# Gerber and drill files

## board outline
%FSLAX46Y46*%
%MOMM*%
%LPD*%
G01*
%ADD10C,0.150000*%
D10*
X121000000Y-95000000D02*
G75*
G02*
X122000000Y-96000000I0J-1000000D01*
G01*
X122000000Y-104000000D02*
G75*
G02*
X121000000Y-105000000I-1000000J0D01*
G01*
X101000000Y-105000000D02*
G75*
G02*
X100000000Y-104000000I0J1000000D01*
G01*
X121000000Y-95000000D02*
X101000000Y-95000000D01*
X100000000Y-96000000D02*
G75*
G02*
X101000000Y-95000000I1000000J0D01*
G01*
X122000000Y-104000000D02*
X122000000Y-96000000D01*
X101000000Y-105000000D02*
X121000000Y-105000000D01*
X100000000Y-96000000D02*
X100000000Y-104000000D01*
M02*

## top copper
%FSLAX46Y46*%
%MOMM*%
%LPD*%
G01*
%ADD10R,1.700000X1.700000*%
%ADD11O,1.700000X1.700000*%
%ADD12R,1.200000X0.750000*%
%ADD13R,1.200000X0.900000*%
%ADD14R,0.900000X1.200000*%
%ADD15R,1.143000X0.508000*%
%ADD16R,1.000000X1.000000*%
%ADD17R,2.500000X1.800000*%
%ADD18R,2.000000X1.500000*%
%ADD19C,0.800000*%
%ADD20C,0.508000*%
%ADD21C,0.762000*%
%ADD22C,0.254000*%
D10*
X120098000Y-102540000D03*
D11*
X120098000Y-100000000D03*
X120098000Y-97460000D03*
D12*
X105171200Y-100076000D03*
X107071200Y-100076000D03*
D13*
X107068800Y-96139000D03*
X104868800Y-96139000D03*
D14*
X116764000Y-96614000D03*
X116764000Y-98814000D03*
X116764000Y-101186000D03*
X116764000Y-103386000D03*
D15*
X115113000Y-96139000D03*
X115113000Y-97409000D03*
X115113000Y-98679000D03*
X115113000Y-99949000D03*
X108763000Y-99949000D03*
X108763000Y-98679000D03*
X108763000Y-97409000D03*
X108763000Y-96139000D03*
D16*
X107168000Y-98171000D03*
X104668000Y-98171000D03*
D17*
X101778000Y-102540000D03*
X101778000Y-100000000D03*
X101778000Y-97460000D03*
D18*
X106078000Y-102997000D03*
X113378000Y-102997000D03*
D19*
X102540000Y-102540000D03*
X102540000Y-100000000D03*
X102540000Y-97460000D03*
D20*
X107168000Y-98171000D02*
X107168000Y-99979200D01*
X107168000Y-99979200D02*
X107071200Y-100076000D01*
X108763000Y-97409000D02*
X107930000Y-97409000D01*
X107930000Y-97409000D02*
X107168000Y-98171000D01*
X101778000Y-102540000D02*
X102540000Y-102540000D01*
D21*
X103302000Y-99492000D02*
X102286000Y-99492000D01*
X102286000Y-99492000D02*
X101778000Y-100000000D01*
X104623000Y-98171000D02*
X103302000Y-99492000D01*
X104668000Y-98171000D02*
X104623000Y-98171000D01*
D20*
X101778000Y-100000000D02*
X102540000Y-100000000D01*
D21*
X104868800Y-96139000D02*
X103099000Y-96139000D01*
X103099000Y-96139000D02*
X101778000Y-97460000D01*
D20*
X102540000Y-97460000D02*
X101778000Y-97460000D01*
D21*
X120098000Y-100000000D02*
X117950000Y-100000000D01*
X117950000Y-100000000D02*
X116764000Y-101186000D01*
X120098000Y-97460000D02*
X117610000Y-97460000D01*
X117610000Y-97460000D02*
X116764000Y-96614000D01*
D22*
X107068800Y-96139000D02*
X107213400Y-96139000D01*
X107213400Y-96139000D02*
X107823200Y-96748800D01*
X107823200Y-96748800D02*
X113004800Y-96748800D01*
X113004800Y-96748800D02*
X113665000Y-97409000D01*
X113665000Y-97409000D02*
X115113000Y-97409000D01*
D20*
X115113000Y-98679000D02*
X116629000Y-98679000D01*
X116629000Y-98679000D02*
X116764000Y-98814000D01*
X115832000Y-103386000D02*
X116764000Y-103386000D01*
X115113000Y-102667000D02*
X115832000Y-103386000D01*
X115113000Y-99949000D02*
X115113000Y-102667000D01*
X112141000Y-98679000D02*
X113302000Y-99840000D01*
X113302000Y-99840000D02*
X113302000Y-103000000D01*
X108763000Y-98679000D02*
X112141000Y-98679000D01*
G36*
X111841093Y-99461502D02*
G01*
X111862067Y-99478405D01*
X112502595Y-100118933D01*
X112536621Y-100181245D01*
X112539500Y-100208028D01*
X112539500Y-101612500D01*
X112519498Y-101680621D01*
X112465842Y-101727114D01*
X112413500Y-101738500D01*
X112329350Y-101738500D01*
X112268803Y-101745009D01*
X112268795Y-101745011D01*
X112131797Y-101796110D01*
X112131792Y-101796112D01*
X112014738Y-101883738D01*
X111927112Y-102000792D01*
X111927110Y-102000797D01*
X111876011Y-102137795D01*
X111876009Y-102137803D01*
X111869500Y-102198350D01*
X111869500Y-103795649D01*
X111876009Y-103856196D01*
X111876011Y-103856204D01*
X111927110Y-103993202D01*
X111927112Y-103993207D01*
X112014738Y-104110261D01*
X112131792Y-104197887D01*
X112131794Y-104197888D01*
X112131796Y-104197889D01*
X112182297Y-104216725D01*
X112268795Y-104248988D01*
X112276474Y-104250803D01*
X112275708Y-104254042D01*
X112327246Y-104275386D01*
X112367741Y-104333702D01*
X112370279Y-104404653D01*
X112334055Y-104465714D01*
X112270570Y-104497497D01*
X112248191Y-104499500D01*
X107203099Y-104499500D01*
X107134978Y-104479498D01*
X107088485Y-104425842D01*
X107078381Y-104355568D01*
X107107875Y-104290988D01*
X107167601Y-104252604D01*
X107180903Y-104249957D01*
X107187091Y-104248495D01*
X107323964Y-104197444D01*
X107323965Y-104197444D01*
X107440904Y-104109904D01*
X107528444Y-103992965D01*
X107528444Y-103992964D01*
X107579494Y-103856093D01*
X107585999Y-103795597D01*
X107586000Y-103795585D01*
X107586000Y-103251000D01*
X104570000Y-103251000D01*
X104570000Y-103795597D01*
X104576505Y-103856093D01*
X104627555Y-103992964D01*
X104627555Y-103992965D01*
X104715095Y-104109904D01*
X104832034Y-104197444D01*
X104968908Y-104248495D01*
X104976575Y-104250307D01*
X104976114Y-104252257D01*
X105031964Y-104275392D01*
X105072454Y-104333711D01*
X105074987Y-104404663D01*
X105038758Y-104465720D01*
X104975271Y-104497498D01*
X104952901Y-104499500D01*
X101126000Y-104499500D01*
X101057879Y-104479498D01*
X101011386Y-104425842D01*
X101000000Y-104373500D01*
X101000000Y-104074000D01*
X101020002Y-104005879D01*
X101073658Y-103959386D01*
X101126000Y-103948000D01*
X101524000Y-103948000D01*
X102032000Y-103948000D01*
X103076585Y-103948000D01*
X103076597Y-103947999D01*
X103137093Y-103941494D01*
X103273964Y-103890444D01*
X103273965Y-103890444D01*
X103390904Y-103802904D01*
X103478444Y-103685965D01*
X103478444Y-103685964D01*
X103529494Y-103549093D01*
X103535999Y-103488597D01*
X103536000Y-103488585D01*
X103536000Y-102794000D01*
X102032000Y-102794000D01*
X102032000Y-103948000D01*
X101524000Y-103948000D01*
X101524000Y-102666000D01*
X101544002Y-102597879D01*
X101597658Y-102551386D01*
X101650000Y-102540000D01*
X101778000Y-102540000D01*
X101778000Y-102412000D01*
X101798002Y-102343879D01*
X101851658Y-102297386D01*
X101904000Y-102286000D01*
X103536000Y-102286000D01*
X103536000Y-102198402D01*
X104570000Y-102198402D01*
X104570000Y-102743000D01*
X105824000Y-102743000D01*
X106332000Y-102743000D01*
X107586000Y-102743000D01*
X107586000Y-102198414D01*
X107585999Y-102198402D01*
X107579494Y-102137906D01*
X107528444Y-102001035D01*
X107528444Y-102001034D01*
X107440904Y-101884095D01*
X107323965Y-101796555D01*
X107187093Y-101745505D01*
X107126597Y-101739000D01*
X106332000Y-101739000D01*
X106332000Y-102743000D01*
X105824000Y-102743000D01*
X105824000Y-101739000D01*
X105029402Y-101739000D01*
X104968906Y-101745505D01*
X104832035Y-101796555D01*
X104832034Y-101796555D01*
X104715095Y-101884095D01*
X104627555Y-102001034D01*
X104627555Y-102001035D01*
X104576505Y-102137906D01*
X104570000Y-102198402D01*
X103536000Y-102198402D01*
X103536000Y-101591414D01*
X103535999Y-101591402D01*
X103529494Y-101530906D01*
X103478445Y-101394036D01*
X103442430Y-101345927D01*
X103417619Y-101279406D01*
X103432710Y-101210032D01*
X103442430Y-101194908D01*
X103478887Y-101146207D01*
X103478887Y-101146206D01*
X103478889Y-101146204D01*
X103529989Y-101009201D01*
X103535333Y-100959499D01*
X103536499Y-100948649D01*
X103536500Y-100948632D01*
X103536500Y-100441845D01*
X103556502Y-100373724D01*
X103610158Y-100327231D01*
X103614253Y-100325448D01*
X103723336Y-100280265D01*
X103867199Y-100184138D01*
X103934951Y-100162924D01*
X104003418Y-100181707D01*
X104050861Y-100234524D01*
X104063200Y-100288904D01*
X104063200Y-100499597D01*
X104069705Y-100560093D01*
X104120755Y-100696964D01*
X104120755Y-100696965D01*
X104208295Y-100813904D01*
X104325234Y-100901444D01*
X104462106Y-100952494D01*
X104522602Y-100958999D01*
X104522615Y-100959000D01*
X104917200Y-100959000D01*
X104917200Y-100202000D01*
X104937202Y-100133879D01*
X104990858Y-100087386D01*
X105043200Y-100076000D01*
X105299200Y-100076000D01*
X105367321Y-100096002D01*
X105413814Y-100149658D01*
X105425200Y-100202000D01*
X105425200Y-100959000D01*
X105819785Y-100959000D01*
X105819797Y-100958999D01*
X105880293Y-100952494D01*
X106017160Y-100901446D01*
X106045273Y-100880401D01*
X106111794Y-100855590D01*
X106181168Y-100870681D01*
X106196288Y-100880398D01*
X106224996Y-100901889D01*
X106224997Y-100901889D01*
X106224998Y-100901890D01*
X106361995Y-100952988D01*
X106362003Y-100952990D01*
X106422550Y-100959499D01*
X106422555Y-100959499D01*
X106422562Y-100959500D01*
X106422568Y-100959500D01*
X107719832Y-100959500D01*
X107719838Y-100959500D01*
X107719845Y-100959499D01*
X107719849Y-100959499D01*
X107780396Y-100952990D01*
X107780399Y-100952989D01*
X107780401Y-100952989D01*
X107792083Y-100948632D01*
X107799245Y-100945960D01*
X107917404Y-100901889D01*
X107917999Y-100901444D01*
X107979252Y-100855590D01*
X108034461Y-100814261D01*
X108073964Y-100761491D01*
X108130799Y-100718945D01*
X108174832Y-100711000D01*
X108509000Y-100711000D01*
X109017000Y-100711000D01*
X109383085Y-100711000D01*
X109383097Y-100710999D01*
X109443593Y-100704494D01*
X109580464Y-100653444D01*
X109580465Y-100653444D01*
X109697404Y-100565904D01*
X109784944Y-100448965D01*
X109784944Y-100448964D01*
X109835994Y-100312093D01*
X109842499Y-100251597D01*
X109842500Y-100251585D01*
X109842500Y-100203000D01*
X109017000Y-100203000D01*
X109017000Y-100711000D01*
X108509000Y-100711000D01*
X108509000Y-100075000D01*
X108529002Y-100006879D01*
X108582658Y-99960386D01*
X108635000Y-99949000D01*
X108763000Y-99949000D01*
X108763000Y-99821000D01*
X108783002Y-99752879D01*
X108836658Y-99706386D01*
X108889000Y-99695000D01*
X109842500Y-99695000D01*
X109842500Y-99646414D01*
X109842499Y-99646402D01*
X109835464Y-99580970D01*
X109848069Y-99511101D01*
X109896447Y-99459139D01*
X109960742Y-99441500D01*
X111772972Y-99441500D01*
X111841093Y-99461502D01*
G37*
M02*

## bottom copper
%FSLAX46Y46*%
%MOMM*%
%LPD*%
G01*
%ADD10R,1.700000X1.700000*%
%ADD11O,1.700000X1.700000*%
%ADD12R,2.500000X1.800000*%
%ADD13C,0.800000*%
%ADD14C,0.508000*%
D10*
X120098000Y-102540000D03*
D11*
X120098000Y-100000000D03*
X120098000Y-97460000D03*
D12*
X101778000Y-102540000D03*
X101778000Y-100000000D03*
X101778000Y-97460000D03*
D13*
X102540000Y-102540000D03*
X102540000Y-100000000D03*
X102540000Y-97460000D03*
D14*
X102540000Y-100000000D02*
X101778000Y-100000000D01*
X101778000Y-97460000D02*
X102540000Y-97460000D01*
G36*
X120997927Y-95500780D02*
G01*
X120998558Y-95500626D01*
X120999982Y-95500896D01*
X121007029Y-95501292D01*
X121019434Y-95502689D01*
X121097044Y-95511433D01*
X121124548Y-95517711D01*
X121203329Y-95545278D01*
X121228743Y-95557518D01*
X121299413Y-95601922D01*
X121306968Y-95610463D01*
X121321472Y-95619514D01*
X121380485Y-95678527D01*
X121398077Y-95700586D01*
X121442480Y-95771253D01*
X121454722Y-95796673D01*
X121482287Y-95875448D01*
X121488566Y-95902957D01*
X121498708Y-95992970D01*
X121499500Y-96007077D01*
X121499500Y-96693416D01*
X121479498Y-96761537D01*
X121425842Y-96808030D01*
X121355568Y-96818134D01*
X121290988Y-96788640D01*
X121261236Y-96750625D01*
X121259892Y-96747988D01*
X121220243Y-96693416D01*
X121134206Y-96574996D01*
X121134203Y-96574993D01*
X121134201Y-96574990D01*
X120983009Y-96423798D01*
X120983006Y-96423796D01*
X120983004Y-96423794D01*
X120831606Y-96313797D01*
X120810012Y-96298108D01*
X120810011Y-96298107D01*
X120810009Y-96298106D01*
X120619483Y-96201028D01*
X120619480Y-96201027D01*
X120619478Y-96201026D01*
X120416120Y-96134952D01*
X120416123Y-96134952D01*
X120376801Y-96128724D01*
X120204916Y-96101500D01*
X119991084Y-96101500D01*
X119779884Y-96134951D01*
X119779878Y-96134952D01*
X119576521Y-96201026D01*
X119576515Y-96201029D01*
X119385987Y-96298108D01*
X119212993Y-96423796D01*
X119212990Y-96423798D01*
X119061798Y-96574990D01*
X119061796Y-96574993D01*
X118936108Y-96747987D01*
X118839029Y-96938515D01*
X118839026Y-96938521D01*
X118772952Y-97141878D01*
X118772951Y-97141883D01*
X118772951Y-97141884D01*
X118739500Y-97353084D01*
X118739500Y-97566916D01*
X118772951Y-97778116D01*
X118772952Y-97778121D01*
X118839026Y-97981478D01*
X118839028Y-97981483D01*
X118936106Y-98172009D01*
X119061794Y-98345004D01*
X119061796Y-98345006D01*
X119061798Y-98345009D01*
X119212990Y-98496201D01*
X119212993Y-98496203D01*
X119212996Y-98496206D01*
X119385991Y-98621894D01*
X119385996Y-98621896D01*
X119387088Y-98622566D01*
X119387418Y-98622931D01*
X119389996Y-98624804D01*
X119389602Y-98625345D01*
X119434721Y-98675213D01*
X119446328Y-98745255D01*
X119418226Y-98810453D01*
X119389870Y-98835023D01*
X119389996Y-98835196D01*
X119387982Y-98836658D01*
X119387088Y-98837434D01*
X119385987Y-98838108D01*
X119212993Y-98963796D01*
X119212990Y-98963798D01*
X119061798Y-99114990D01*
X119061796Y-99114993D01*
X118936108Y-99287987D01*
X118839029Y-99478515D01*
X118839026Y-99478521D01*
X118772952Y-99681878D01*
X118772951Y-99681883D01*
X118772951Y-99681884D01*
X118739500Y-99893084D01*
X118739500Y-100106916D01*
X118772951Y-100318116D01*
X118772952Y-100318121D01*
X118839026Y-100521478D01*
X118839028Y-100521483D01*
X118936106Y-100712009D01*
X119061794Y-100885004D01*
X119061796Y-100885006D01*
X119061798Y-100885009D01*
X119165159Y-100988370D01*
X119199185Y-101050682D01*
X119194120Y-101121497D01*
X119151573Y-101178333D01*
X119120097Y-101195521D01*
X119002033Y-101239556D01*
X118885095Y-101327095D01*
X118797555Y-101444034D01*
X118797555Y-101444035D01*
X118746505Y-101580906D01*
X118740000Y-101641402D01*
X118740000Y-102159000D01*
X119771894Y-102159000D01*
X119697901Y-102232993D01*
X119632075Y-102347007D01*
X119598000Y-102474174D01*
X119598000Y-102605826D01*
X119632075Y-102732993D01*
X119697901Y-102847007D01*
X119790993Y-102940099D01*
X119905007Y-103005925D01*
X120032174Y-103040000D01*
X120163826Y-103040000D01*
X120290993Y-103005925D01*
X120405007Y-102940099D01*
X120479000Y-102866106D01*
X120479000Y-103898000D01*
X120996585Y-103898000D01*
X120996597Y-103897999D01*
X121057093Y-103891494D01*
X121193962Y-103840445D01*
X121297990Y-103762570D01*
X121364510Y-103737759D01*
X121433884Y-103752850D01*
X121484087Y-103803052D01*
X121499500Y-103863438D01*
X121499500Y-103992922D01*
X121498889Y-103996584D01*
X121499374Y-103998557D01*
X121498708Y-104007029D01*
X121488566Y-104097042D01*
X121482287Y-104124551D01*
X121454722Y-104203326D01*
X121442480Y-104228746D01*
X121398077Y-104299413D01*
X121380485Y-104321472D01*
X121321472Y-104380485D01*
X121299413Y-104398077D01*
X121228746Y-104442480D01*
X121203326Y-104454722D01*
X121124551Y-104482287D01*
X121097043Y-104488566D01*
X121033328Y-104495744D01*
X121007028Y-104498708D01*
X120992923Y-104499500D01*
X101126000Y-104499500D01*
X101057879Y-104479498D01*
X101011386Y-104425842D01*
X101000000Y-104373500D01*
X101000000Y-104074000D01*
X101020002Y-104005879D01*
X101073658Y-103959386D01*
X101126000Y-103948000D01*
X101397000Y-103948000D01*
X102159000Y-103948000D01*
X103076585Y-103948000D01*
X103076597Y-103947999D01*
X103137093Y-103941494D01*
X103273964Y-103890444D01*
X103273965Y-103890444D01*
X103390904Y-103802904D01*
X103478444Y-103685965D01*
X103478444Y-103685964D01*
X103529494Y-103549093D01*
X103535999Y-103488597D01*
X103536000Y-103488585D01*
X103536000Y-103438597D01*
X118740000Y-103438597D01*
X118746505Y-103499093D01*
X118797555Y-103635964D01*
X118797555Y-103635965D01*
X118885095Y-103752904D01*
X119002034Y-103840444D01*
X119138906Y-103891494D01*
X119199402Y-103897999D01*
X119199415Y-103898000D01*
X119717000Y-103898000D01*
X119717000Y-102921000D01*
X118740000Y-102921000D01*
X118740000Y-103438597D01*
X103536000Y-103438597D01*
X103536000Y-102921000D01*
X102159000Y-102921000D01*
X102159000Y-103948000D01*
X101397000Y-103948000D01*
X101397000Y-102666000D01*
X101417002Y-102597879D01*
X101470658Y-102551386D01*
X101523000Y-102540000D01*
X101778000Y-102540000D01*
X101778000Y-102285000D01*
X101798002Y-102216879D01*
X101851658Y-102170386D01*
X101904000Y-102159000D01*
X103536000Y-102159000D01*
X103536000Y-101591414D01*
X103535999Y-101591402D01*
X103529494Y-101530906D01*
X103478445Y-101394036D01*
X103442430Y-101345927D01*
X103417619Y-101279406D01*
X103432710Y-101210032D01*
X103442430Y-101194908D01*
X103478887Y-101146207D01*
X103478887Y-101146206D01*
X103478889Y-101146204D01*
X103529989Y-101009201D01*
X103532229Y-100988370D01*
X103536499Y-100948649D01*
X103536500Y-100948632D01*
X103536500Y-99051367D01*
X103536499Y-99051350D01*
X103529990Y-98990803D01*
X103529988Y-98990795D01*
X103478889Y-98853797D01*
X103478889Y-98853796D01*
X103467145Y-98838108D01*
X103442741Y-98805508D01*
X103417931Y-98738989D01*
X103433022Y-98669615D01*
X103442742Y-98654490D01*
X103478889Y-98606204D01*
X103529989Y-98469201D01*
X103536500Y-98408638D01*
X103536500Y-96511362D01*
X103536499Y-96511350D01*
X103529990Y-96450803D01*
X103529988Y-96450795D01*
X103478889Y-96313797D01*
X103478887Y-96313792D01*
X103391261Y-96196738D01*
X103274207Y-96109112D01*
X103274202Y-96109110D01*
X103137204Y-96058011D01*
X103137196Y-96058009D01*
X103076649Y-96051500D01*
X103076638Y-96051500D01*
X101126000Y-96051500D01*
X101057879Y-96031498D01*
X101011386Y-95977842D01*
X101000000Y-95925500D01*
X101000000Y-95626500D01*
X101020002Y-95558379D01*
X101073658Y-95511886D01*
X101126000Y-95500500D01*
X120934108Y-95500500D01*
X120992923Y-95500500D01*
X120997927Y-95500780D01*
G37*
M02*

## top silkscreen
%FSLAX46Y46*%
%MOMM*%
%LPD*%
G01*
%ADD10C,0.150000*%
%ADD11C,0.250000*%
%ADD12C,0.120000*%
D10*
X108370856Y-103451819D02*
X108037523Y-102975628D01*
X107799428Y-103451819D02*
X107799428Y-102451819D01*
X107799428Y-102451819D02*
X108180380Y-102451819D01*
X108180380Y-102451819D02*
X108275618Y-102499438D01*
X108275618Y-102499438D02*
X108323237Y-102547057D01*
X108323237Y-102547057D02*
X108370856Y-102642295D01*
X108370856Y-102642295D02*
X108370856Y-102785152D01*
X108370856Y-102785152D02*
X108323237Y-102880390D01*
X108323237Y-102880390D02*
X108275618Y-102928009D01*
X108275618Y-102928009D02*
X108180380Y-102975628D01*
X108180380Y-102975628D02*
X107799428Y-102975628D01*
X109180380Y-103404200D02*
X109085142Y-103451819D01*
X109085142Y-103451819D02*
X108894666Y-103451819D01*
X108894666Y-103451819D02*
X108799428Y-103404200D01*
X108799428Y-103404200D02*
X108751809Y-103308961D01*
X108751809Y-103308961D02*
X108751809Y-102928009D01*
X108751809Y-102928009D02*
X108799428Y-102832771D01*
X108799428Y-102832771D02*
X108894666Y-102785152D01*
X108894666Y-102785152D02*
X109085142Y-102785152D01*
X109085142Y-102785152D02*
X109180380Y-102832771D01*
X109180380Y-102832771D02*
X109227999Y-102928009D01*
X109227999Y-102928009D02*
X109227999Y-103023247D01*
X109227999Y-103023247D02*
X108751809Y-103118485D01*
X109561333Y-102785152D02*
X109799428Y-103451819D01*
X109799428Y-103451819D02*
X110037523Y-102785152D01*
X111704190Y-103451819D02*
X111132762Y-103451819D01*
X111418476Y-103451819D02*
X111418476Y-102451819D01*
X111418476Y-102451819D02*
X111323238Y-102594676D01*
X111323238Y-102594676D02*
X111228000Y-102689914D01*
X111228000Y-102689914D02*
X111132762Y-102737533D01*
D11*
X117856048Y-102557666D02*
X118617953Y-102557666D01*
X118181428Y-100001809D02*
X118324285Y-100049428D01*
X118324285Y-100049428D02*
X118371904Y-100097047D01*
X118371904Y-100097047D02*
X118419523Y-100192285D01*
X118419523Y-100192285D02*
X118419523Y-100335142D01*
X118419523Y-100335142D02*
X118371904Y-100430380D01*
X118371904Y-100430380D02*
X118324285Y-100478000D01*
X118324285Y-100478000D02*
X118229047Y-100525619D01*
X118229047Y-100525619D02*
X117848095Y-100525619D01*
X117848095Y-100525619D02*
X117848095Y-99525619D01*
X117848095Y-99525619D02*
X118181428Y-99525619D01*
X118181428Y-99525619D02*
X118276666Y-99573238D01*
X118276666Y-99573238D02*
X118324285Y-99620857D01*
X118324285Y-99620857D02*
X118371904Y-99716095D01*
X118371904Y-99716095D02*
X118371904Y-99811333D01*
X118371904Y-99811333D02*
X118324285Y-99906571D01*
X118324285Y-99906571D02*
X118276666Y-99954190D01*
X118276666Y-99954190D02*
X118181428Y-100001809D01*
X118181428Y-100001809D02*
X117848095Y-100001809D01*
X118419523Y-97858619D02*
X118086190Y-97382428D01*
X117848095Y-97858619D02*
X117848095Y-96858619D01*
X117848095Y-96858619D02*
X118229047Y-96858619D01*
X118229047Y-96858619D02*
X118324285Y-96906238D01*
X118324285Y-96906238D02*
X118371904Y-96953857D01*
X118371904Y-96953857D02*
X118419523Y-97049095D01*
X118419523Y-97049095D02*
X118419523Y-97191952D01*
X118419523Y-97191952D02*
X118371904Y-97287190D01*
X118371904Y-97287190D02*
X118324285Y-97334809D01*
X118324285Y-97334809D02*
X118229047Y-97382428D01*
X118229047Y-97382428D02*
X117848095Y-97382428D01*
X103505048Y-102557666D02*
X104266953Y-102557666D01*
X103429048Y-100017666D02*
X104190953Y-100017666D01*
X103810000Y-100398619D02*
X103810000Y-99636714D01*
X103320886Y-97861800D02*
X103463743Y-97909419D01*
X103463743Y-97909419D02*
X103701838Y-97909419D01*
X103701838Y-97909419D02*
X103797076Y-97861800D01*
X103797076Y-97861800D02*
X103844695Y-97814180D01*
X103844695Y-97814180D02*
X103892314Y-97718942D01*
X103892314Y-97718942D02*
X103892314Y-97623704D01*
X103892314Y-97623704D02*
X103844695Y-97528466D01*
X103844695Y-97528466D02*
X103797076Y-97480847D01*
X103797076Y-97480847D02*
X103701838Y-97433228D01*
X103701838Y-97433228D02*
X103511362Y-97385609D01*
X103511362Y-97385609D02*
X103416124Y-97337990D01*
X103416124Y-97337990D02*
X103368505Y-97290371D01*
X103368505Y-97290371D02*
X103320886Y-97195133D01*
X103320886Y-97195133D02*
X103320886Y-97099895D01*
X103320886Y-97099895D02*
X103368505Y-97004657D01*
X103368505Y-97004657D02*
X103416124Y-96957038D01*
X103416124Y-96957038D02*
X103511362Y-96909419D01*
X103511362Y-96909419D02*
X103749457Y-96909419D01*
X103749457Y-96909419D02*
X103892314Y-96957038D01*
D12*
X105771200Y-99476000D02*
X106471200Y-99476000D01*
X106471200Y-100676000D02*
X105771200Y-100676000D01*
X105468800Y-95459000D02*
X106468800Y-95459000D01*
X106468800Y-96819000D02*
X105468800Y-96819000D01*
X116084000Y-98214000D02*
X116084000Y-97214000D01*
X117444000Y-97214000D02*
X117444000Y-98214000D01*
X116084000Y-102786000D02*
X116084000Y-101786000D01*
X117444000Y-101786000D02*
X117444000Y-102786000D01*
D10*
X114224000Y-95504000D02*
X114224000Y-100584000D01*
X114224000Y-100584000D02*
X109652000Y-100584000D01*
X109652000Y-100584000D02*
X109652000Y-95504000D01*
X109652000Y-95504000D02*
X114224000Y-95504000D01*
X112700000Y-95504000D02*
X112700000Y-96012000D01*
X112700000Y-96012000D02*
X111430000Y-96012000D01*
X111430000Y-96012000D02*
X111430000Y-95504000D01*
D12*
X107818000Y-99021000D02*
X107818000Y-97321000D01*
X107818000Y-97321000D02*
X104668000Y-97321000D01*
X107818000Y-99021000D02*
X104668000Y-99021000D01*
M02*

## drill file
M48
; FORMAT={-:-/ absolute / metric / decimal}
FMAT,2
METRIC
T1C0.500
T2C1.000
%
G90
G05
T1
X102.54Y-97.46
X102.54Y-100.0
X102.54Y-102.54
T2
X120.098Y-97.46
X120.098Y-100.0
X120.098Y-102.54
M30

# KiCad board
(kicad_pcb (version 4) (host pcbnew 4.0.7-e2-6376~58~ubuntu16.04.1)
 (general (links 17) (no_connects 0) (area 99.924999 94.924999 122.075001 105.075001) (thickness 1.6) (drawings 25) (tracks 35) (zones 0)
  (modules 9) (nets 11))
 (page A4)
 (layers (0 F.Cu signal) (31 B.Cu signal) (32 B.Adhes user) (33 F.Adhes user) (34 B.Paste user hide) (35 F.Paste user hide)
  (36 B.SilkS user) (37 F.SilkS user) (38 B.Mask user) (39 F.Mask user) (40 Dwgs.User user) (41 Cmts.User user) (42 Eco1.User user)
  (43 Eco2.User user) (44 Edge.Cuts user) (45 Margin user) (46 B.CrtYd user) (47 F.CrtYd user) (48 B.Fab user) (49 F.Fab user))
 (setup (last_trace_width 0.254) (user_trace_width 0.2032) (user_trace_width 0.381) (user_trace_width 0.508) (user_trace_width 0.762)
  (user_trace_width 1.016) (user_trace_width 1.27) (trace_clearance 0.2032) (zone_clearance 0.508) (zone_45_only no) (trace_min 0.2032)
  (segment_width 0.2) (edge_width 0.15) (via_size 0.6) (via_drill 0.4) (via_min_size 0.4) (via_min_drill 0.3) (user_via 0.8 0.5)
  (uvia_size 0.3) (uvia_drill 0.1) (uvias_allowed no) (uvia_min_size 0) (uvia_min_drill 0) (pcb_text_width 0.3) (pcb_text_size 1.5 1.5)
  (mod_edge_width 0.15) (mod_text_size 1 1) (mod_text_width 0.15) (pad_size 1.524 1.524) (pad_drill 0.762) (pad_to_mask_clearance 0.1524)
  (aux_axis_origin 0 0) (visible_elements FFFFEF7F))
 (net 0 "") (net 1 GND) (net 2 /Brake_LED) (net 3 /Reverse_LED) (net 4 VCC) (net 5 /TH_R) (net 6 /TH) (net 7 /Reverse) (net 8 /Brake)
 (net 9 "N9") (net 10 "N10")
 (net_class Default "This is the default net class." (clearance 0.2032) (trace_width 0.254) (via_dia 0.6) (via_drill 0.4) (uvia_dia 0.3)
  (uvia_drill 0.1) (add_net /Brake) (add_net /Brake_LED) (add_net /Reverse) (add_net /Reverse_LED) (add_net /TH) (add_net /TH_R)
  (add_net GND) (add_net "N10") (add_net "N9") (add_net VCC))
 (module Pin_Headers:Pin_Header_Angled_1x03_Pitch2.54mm (layer B.Cu) (at 120.098 102.54)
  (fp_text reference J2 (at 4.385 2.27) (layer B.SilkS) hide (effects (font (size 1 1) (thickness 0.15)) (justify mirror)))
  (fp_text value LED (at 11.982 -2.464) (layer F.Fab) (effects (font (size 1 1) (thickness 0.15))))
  (pad 1 thru_hole rect (at 0 0) (size 1.7 1.7) (drill 1) (layers *.Cu *.Mask) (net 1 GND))
  (pad 2 thru_hole oval (at 0 -2.54) (size 1.7 1.7) (drill 1) (layers *.Cu *.Mask) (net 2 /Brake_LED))
  (pad 3 thru_hole oval (at 0 -5.08) (size 1.7 1.7) (drill 1) (layers *.Cu *.Mask) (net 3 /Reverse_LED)))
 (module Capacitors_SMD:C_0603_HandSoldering (layer F.Cu) (at 106.1212 100.076)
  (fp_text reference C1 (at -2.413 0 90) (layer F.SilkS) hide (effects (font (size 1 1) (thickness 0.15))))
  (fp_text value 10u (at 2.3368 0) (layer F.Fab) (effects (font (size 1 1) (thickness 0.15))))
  (fp_line (start -0.35 -0.6) (end 0.35 -0.6) (layer F.SilkS) (width 0.12))
  (fp_line (start 0.35 0.6) (end -0.35 0.6) (layer F.SilkS) (width 0.12))
  (pad 1 smd rect (at -0.95 0) (size 1.2 0.75) (layers F.Cu F.Paste F.Mask) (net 1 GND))
  (pad 2 smd rect (at 0.95 0) (size 1.2 0.75) (layers F.Cu F.Paste F.Mask) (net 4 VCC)))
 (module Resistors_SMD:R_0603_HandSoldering (layer F.Cu) (at 105.9688 96.139 180)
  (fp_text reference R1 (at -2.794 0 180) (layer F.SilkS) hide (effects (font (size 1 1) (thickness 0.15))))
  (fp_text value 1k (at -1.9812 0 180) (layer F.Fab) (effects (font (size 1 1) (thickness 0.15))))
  (fp_line (start 0.5 0.68) (end -0.5 0.68) (layer F.SilkS) (width 0.12))
  (fp_line (start -0.5 -0.68) (end 0.5 -0.68) (layer F.SilkS) (width 0.12))
  (pad 1 smd rect (at -1.1 0 180) (size 1.2 0.9) (layers F.Cu F.Paste F.Mask) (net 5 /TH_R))
  (pad 2 smd rect (at 1.1 0 180) (size 1.2 0.9) (layers F.Cu F.Paste F.Mask) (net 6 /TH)))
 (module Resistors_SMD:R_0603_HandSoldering (layer F.Cu) (at 116.764 97.714 270)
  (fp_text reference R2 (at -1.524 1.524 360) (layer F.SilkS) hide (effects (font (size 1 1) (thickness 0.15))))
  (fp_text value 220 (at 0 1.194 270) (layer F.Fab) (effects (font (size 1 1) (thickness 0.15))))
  (fp_line (start 0.5 0.68) (end -0.5 0.68) (layer F.SilkS) (width 0.12))
  (fp_line (start -0.5 -0.68) (end 0.5 -0.68) (layer F.SilkS) (width 0.12))
  (pad 1 smd rect (at -1.1 0 270) (size 1.2 0.9) (layers F.Cu F.Paste F.Mask) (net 3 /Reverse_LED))
  (pad 2 smd rect (at 1.1 0 270) (size 1.2 0.9) (layers F.Cu F.Paste F.Mask) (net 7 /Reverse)))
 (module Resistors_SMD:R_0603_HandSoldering (layer F.Cu) (at 116.764 102.286 270)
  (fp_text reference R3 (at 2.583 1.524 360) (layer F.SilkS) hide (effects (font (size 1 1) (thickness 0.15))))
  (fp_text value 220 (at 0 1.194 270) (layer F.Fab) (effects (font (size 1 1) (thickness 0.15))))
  (fp_line (start 0.5 0.68) (end -0.5 0.68) (layer F.SilkS) (width 0.12))
  (fp_line (start -0.5 -0.68) (end 0.5 -0.68) (layer F.SilkS) (width 0.12))
  (pad 1 smd rect (at -1.1 0 270) (size 1.2 0.9) (layers F.Cu F.Paste F.Mask) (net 2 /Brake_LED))
  (pad 2 smd rect (at 1.1 0 270) (size 1.2 0.9) (layers F.Cu F.Paste F.Mask) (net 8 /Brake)))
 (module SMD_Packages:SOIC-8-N (layer F.Cu) (at 111.938 98.044 270)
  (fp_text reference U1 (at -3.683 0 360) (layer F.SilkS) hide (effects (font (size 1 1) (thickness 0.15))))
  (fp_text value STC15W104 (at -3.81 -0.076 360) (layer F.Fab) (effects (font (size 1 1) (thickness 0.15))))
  (fp_line (start -2.54 -2.286) (end 2.54 -2.286) (layer F.SilkS) (width 0.15))
  (fp_line (start 2.54 -2.286) (end 2.54 2.286) (layer F.SilkS) (width 0.15))
  (fp_line (start 2.54 2.286) (end -2.54 2.286) (layer F.SilkS) (width 0.15))
  (fp_line (start -2.54 2.286) (end -2.54 -2.286) (layer F.SilkS) (width 0.15))
  (fp_line (start -2.54 -0.762) (end -2.032 -0.762) (layer F.SilkS) (width 0.15))
  (fp_line (start -2.032 -0.762) (end -2.032 0.508) (layer F.SilkS) (width 0.15))
  (fp_line (start -2.032 0.508) (end -2.54 0.508) (layer F.SilkS) (width 0.15))
  (pad 8 smd rect (at -1.905 -3.175 270) (size 0.508 1.143) (layers F.Cu F.Paste F.Mask))
  (pad 7 smd rect (at -0.635 -3.175 270) (size 0.508 1.143) (layers F.Cu F.Paste F.Mask) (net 5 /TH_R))
  (pad 6 smd rect (at 0.635 -3.175 270) (size 0.508 1.143) (layers F.Cu F.Paste F.Mask) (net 7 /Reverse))
  (pad 5 smd rect (at 1.905 -3.175 270) (size 0.508 1.143) (layers F.Cu F.Paste F.Mask) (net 8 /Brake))
  (pad 4 smd rect (at 1.905 3.175 270) (size 0.508 1.143) (layers F.Cu F.Paste F.Mask) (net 1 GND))
  (pad 3 smd rect (at 0.635 3.175 270) (size 0.508 1.143) (layers F.Cu F.Paste F.Mask) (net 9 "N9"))
  (pad 2 smd rect (at -0.635 3.175 270) (size 0.508 1.143) (layers F.Cu F.Paste F.Mask) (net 4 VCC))
  (pad 1 smd rect (at -1.905 3.175 270) (size 0.508 1.143) (layers F.Cu F.Paste F.Mask)))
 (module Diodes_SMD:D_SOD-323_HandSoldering (layer F.Cu) (at 105.918 98.171 180)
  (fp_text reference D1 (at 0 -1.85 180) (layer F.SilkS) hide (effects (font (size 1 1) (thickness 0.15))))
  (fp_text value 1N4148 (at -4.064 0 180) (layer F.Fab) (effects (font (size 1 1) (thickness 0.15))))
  (fp_line (start -1.9 -0.85) (end -1.9 0.85) (layer F.SilkS) (width 0.12))
  (fp_line (start -1.9 0.85) (end 1.25 0.85) (layer F.SilkS) (width 0.12))
  (fp_line (start -1.9 -0.85) (end 1.25 -0.85) (layer F.SilkS) (width 0.12))
  (pad 1 smd rect (at -1.25 0 180) (size 1 1) (layers F.Cu F.Paste F.Mask) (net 4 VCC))
  (pad 2 smd rect (at 1.25 0 180) (size 1 1) (layers F.Cu F.Paste F.Mask) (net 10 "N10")))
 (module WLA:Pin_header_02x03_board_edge (layer F.Cu) (at 100 100)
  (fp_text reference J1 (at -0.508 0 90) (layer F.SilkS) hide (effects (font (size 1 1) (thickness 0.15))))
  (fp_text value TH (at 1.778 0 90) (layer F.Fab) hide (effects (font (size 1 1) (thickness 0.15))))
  (pad 1 smd rect (at 1.778 2.54) (size 2.5 1.8) (layers F.Cu F.Mask) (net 1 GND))
  (pad 2 smd rect (at 1.778 2.54) (size 2.5 1.8) (layers B.Cu B.Mask) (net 1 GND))
  (pad 3 smd rect (at 1.778 0) (size 2.5 1.8) (layers F.Cu F.Mask) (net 10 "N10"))
  (pad 4 smd rect (at 1.778 0) (size 2.5 1.8) (layers B.Cu B.Mask) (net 10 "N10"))
  (pad 5 smd rect (at 1.778 -2.54) (size 2.5 1.8) (layers F.Cu F.Mask) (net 6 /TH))
  (pad 6 smd rect (at 1.778 -2.54) (size 2.5 1.8) (layers B.Cu B.Mask) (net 6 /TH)))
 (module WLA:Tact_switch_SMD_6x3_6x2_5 (layer F.Cu) (at 109.728 102.997)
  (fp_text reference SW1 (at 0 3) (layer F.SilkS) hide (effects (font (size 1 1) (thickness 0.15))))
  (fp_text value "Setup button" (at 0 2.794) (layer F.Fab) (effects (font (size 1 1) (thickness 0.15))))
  (pad 1 smd rect (at -3.65 0) (size 2 1.5) (layers F.Cu F.Paste F.Mask) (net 1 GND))
  (pad 2 smd rect (at 3.65 0) (size 2 1.5) (layers F.Cu F.Paste F.Mask) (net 9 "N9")))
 (gr_arc (start 121 96) (end 121 95) (angle 90) (layer Edge.Cuts) (width 0.15))
 (gr_arc (start 121 104) (end 122 104) (angle 90) (layer Edge.Cuts) (width 0.15))
 (gr_arc (start 101 104) (end 101 105) (angle 90) (layer Edge.Cuts) (width 0.15))
 (gr_line (start 121 95) (end 101 95) (layer Edge.Cuts) (width 0.15))
 (gr_arc (start 101 96) (end 100 96) (angle 90) (layer Edge.Cuts) (width 0.15))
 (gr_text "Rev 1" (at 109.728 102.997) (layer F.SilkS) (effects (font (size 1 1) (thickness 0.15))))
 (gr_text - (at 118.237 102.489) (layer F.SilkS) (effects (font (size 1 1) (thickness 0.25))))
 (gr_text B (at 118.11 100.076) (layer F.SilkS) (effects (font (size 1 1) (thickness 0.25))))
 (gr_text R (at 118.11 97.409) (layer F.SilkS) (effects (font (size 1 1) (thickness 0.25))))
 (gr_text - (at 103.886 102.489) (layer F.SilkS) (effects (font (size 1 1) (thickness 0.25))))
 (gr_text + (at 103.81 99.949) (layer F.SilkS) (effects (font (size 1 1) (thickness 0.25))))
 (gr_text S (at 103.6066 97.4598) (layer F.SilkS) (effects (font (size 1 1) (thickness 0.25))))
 (gr_line (start 122 104) (end 122 96) (layer Edge.Cuts) (width 0.15))
 (gr_line (start 101 105) (end 121 105) (layer Edge.Cuts) (width 0.15))
 (gr_line (start 100 96) (end 100 104) (layer Edge.Cuts) (width 0.15))
 (segment (start 107.168 98.171) (end 107.168 99.9792) (width 0.508) (layer F.Cu) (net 4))
 (segment (start 107.168 99.9792) (end 107.0712 100.076) (width 0.508) (layer F.Cu) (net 4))
 (segment (start 108.763 97.409) (end 107.93 97.409) (width 0.508) (layer F.Cu) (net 4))
 (segment (start 107.93 97.409) (end 107.168 98.171) (width 0.508) (layer F.Cu) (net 4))
 (via (at 102.54 102.54) (size 0.8) (drill 0.5) (layers F.Cu B.Cu) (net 1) (status 30))
 (segment (start 101.778 102.54) (end 102.54 102.54) (width 0.508) (layer F.Cu) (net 1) (status 30))
 (segment (start 103.302 99.492) (end 102.286 99.492) (width 0.762) (layer F.Cu) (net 10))
 (segment (start 102.286 99.492) (end 101.778 100) (width 0.762) (layer F.Cu) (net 10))
 (segment (start 104.623 98.171) (end 103.302 99.492) (width 0.762) (layer F.Cu) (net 10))
 (segment (start 104.668 98.171) (end 104.623 98.171) (width 0.762) (layer F.Cu) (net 10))
 (via (at 102.54 100) (size 0.8) (drill 0.5) (layers F.Cu B.Cu) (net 10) (status 30))
 (segment (start 102.54 100) (end 101.778 100) (width 0.508) (layer B.Cu) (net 10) (status 30))
 (segment (start 101.778 100) (end 102.54 100) (width 0.508) (layer F.Cu) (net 10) (status 30))
 (segment (start 104.8688 96.139) (end 103.099 96.139) (width 0.762) (layer F.Cu) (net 6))
 (segment (start 103.099 96.139) (end 101.778 97.46) (width 0.762) (layer F.Cu) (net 6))
 (via (at 102.54 97.46) (size 0.8) (drill 0.5) (layers F.Cu B.Cu) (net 6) (status 30))
 (segment (start 102.54 97.46) (end 101.778 97.46) (width 0.508) (layer F.Cu) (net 6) (status 30))
 (segment (start 101.778 97.46) (end 102.54 97.46) (width 0.508) (layer B.Cu) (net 6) (status 30))
 (segment (start 120.098 100) (end 117.95 100) (width 0.762) (layer F.Cu) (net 2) (status 10))
 (segment (start 117.95 100) (end 116.764 101.186) (width 0.762) (layer F.Cu) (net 2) (status 20))
 (segment (start 120.098 97.46) (end 117.61 97.46) (width 0.762) (layer F.Cu) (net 3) (status 10))
 (segment (start 117.61 97.46) (end 116.764 96.614) (width 0.762) (layer F.Cu) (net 3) (status 20))
 (segment (start 107.0688 96.139) (end 107.2134 96.139) (width 0.254) (layer F.Cu) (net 5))
 (segment (start 107.2134 96.139) (end 107.8232 96.7488) (width 0.254) (layer F.Cu) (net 5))
 (segment (start 107.8232 96.7488) (end 113.0048 96.7488) (width 0.254) (layer F.Cu) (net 5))
 (segment (start 113.0048 96.7488) (end 113.665 97.409) (width 0.254) (layer F.Cu) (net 5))
 (segment (start 113.665 97.409) (end 115.113 97.409) (width 0.254) (layer F.Cu) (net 5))
 (segment (start 115.113 98.679) (end 116.629 98.679) (width 0.508) (layer F.Cu) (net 7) (status 30))
 (segment (start 116.629 98.679) (end 116.764 98.814) (width 0.508) (layer F.Cu) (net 7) (status 30))
 (segment (start 115.832 103.386) (end 116.764 103.386) (width 0.508) (layer F.Cu) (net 8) (status 20))
 (segment (start 115.113 102.667) (end 115.832 103.386) (width 0.508) (layer F.Cu) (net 8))
 (segment (start 115.113 99.949) (end 115.113 102.667) (width 0.508) (layer F.Cu) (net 8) (status 10))
 (segment (start 112.141 98.679) (end 113.302 99.84) (width 0.508) (layer F.Cu) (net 9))
 (segment (start 113.302 99.84) (end 113.302 103) (width 0.508) (layer F.Cu) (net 9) (status 20))
 (segment (start 108.763 98.679) (end 112.141 98.679) (width 0.508) (layer F.Cu) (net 9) (status 10))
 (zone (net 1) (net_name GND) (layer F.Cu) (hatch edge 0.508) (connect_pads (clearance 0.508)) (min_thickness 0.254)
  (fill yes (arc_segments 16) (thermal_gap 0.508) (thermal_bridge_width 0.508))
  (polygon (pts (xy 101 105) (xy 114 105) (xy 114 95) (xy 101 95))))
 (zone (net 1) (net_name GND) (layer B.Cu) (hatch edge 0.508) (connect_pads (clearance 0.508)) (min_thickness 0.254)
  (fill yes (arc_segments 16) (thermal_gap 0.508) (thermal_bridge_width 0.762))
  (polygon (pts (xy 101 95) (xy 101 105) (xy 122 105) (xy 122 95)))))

